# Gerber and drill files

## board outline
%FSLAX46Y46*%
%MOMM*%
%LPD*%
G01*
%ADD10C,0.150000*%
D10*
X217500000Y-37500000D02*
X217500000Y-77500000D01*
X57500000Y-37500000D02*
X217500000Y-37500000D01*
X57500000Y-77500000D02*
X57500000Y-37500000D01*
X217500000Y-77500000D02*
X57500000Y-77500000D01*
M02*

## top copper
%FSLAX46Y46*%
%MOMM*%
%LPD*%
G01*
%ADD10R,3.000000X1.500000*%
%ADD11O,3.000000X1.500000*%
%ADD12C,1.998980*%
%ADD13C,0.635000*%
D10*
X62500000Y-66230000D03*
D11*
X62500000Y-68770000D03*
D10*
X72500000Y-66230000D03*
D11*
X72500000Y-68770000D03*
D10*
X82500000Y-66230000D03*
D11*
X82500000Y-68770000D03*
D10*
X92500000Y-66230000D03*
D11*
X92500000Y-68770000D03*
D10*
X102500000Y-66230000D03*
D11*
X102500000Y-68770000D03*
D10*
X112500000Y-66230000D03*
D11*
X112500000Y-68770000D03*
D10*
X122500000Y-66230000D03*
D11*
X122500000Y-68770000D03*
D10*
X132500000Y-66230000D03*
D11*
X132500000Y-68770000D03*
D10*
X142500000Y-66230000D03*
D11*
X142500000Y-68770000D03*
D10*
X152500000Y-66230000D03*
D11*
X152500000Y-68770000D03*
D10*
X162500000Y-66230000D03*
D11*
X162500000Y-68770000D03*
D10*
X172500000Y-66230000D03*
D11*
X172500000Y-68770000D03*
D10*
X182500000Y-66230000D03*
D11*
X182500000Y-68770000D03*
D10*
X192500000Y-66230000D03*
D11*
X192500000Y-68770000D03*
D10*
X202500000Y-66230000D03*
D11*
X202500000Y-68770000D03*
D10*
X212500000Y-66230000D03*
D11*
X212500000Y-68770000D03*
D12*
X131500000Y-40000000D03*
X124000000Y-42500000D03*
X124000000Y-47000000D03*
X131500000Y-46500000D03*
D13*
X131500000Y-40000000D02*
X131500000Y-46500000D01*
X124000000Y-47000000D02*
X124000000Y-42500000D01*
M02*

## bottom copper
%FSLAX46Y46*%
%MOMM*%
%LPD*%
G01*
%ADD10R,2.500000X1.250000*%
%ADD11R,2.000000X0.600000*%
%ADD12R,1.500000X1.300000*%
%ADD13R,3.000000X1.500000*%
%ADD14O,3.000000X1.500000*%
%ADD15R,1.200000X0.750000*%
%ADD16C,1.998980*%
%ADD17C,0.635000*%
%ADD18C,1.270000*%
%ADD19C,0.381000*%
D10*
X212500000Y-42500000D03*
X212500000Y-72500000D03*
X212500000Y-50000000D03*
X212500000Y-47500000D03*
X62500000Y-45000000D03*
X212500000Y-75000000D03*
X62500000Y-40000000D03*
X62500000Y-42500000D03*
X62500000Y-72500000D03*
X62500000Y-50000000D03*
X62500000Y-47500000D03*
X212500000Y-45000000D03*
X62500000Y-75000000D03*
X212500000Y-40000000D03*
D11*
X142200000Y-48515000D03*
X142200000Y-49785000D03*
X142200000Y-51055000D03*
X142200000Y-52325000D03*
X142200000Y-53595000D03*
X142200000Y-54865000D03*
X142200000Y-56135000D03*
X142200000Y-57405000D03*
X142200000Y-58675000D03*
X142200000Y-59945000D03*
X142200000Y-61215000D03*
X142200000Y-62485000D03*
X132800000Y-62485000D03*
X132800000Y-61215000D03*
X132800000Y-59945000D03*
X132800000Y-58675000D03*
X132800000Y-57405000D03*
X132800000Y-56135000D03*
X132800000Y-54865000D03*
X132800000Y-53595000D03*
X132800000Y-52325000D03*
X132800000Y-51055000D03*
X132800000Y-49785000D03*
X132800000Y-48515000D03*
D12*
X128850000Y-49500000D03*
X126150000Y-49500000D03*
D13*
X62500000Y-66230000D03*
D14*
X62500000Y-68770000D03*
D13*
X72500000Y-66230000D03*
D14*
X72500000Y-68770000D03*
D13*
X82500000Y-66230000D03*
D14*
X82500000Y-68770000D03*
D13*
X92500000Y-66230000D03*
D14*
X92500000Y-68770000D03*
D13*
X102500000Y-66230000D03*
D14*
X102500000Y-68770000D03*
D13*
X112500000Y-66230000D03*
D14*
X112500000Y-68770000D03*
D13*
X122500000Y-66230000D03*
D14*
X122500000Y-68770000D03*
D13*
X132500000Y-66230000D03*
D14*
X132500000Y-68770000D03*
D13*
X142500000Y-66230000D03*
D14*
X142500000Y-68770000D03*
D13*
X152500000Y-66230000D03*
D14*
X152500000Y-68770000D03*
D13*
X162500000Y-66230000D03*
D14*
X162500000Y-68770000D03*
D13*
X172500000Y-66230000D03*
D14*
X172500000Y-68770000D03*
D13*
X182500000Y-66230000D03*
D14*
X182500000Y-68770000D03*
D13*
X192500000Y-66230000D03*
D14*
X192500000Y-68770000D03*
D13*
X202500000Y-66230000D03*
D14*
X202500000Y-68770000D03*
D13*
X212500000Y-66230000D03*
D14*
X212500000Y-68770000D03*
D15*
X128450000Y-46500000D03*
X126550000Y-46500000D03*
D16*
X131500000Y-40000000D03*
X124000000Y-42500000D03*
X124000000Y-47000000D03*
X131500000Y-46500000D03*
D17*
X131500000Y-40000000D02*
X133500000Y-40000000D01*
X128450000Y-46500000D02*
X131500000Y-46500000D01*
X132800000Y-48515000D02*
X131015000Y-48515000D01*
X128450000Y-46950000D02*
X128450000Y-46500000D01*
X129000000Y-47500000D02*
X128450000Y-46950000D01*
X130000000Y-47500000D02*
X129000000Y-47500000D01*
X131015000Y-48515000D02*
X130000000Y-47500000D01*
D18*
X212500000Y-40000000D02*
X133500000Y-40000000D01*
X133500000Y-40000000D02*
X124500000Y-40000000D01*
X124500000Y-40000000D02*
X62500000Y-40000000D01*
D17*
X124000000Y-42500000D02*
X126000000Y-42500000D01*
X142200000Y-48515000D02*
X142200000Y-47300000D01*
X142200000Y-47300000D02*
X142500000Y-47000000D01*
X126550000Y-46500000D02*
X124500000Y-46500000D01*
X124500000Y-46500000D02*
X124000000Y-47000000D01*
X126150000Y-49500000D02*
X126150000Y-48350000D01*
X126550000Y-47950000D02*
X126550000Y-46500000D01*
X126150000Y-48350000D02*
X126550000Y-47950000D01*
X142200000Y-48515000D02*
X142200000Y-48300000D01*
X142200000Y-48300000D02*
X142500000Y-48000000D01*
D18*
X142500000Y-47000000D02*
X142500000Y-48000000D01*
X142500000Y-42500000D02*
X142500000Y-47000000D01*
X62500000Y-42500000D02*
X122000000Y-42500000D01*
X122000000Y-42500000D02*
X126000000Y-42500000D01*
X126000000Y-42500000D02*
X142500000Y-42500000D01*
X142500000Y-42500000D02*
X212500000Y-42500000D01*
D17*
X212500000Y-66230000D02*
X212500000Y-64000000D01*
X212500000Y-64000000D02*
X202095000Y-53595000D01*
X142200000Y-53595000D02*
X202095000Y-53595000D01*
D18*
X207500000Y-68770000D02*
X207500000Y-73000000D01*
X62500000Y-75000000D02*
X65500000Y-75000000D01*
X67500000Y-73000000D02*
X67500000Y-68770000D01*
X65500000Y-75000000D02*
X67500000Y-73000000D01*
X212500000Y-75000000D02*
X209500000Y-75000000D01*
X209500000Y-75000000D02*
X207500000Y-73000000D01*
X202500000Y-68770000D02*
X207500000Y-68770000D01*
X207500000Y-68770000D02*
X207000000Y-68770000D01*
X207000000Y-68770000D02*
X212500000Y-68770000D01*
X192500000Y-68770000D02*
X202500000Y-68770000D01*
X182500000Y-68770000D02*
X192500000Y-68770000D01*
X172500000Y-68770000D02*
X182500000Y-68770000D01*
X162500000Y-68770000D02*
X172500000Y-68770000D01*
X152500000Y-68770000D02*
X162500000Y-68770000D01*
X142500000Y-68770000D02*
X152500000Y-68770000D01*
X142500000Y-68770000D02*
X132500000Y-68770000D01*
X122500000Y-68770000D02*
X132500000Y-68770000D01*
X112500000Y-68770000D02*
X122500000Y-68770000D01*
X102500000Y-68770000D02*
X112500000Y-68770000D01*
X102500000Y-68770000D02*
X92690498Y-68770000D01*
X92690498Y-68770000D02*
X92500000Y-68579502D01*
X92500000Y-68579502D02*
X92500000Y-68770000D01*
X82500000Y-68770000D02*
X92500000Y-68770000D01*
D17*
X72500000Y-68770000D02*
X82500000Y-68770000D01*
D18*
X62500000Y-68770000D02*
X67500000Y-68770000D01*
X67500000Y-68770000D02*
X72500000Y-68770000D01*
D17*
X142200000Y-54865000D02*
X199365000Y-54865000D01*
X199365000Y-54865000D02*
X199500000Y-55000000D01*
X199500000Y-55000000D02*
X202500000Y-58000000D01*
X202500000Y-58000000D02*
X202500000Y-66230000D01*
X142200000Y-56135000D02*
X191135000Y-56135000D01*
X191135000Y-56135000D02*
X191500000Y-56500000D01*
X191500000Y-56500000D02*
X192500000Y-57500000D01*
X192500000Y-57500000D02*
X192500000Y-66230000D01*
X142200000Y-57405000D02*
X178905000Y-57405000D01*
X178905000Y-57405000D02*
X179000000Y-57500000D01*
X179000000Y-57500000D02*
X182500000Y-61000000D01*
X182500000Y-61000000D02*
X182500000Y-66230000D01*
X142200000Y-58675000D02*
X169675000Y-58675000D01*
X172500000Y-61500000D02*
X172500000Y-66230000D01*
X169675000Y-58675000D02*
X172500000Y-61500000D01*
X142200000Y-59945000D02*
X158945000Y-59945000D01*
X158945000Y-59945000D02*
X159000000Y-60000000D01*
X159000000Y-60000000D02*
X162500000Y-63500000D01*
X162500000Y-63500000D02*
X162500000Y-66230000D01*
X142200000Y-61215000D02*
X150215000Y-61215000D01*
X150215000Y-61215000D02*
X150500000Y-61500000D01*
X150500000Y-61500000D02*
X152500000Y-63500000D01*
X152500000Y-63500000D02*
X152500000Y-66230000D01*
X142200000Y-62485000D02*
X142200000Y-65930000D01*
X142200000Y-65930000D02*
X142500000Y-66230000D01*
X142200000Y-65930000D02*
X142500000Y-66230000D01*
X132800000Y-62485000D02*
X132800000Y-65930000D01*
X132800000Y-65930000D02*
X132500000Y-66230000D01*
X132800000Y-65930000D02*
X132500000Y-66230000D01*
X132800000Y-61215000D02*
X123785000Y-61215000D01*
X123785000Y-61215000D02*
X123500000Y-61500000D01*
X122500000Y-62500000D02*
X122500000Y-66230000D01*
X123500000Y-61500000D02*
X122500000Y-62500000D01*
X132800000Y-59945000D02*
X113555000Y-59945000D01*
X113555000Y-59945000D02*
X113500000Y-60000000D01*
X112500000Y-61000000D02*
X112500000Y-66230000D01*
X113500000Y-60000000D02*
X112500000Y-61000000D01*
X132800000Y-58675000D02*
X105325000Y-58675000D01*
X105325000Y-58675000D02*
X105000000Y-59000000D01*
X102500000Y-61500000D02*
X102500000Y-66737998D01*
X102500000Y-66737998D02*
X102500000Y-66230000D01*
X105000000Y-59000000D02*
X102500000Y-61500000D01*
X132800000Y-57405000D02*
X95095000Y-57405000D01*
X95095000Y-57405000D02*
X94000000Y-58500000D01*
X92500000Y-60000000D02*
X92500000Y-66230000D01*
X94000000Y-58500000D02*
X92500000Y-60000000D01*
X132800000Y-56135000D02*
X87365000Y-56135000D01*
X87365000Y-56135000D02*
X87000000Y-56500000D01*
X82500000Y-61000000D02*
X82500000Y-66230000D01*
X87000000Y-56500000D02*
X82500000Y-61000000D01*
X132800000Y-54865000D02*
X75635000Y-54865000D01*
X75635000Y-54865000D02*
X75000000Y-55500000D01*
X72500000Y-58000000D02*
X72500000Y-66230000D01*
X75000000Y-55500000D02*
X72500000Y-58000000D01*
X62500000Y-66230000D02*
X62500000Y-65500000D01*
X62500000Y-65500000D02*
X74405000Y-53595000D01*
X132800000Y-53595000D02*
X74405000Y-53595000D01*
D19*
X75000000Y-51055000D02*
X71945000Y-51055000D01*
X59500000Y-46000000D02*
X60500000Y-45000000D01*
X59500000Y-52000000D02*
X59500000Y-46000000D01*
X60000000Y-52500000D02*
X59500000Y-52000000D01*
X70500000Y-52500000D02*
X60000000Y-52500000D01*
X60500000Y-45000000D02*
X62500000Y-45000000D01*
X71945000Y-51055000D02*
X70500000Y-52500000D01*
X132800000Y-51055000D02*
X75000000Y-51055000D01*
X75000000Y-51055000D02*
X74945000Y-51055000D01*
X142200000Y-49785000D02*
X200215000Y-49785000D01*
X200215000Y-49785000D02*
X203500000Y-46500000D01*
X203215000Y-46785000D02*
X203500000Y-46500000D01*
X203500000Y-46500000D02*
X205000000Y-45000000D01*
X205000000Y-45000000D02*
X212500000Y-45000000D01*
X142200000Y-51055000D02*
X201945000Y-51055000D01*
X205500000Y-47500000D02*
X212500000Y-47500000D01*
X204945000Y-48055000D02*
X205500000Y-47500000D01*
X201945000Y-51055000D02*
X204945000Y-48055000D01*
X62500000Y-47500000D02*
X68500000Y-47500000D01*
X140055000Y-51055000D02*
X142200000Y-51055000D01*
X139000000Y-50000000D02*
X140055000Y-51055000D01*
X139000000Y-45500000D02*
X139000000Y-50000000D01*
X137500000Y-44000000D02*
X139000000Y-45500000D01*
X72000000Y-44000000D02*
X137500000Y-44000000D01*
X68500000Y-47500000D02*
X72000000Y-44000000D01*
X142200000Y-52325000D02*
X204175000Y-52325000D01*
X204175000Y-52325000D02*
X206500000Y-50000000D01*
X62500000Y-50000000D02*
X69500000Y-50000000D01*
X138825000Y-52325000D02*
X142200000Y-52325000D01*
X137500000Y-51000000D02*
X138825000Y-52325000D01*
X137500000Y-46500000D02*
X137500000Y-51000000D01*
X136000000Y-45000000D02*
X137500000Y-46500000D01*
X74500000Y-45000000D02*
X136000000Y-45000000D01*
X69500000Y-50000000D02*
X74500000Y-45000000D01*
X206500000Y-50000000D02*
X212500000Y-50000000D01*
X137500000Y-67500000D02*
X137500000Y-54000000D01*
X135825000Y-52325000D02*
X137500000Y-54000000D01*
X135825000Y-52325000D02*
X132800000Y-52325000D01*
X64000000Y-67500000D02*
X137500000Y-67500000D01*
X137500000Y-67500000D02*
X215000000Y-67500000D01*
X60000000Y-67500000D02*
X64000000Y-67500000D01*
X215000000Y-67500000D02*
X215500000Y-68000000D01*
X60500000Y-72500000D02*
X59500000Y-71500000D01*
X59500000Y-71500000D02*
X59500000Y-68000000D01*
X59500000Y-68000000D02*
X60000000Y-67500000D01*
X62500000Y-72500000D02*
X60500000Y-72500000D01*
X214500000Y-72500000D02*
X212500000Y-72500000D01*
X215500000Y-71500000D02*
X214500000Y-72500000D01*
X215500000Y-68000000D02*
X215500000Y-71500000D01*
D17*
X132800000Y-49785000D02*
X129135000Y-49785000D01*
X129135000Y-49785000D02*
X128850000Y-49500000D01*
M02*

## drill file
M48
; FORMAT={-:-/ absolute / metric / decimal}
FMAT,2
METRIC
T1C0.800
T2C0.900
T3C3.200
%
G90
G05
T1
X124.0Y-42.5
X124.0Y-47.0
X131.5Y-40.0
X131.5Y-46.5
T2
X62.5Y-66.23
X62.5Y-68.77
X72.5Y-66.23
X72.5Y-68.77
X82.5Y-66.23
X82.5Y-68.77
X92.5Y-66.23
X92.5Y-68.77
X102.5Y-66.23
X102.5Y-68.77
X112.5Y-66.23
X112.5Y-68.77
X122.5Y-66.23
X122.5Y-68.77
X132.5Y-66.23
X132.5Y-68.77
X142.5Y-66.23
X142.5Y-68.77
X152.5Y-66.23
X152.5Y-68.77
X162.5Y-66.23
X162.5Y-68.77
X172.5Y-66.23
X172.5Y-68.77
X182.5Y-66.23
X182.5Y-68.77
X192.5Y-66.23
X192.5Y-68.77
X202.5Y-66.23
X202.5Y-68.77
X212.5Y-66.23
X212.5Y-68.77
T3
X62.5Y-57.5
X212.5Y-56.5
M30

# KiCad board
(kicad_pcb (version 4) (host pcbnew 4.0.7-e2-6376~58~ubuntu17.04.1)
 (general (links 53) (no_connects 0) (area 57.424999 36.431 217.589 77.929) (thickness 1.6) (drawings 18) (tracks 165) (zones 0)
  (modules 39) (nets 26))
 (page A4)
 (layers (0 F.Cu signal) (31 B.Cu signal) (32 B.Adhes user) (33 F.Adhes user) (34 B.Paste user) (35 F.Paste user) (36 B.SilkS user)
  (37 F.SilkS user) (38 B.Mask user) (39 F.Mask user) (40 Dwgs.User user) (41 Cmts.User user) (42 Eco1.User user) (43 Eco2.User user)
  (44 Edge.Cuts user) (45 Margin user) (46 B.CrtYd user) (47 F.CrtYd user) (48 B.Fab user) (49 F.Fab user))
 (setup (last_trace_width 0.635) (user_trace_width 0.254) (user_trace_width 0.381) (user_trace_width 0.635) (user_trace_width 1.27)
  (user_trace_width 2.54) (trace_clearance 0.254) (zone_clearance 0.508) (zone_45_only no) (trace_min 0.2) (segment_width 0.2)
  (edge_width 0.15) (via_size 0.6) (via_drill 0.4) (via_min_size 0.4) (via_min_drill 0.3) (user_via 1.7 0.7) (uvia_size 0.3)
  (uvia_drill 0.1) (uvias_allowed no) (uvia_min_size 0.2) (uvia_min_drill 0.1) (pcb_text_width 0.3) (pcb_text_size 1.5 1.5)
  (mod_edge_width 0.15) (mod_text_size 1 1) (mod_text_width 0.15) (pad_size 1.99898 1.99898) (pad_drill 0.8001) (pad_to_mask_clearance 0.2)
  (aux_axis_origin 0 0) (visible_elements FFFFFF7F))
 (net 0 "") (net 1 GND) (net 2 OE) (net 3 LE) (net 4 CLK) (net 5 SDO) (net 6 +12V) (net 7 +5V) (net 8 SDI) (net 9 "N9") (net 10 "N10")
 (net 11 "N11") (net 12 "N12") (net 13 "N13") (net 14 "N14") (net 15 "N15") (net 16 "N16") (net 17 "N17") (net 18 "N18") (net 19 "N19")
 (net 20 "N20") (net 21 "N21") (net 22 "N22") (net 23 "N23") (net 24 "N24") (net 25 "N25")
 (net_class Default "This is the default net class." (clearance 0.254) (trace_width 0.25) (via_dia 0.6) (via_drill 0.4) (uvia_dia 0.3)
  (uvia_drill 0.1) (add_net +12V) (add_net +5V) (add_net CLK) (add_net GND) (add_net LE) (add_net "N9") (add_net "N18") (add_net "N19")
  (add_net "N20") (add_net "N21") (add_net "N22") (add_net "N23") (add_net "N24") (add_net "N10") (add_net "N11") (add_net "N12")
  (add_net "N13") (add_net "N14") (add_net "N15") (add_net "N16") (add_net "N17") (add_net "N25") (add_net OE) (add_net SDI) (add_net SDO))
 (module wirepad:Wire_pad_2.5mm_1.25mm (layer B.Cu) (at 212.5 42.5 180)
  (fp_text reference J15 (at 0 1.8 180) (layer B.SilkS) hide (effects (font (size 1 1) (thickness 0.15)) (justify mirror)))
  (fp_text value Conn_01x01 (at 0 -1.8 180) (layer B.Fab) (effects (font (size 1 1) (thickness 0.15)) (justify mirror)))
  (pad 1 smd rect (at 0 0 180) (size 2.5 1.25) (layers B.Cu B.Mask) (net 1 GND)))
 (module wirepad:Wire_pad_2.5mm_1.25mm (layer B.Cu) (at 212.5 72.5 180)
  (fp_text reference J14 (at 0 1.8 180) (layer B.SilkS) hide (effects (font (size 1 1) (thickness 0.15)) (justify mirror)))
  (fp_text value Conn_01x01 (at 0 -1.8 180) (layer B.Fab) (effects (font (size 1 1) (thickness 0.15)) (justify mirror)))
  (pad 1 smd rect (at 0 0 180) (size 2.5 1.25) (layers B.Cu B.Mask) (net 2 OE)))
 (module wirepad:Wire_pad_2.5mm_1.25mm (layer B.Cu) (at 212.5 50 180)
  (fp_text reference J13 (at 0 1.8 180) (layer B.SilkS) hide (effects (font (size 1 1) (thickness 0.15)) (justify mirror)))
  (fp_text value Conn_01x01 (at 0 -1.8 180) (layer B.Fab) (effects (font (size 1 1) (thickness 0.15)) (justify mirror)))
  (pad 1 smd rect (at 0 0 180) (size 2.5 1.25) (layers B.Cu B.Mask) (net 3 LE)))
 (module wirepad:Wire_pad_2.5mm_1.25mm (layer B.Cu) (at 212.5 47.5 180)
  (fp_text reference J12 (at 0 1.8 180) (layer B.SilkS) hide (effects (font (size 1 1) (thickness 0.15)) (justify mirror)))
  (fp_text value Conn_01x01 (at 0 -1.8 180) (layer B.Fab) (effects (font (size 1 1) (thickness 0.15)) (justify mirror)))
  (pad 1 smd rect (at 0 0 180) (size 2.5 1.25) (layers B.Cu B.Mask) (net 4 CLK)))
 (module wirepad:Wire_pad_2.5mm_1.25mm (layer B.Cu) (at 62.5 45 180)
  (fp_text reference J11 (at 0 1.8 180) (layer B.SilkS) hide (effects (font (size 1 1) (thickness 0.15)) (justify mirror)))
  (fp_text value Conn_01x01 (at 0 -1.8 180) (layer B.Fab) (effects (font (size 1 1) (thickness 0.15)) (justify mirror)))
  (pad 1 smd rect (at 0 0 180) (size 2.5 1.25) (layers B.Cu B.Mask) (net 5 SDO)))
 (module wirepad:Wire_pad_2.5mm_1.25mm (layer B.Cu) (at 212.5 75 180)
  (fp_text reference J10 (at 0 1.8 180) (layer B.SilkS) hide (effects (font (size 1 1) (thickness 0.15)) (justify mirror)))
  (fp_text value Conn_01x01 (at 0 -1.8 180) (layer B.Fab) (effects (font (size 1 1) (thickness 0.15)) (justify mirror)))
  (pad 1 smd rect (at 0 0 180) (size 2.5 1.25) (layers B.Cu B.Mask) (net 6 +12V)))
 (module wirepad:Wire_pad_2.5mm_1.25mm (layer B.Cu) (at 62.5 40 180)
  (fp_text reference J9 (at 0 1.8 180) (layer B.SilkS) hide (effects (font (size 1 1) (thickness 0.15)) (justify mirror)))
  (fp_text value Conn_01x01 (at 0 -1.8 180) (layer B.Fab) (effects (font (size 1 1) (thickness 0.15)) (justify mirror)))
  (pad 1 smd rect (at 0 0 180) (size 2.5 1.25) (layers B.Cu B.Mask) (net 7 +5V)))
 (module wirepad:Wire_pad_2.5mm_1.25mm (layer B.Cu) (at 62.5 42.5 180)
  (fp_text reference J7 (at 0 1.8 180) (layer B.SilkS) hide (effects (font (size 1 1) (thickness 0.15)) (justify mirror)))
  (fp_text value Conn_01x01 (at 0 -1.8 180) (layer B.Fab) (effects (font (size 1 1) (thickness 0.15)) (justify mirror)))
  (pad 1 smd rect (at 0 0 180) (size 2.5 1.25) (layers B.Cu B.Mask) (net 1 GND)))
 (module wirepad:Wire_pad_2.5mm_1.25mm (layer B.Cu) (at 62.5 72.5 180)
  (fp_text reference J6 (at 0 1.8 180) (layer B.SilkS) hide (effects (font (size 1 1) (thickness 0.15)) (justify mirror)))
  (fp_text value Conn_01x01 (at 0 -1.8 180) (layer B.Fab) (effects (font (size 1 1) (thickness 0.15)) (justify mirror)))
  (pad 1 smd rect (at 0 0 180) (size 2.5 1.25) (layers B.Cu B.Mask) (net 2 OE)))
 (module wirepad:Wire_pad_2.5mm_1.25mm (layer B.Cu) (at 62.5 50 180)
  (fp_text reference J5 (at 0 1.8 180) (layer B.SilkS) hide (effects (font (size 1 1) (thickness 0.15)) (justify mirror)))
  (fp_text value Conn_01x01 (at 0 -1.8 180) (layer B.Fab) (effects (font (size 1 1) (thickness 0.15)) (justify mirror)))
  (pad 1 smd rect (at 0 0 180) (size 2.5 1.25) (layers B.Cu B.Mask) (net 3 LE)))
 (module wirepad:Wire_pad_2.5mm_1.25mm (layer B.Cu) (at 62.5 47.5 180)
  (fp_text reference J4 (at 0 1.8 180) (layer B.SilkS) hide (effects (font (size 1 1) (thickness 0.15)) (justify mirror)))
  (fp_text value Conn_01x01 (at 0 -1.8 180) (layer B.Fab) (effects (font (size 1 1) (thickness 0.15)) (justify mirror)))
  (pad 1 smd rect (at 0 0 180) (size 2.5 1.25) (layers B.Cu B.Mask) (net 4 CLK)))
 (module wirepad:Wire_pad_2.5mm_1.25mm (layer B.Cu) (at 212.5 45 180)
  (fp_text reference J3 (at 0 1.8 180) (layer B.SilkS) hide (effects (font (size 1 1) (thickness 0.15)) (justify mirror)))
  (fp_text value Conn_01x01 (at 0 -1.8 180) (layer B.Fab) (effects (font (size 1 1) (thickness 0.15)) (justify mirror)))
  (pad 1 smd rect (at 0 0 180) (size 2.5 1.25) (layers B.Cu B.Mask) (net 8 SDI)))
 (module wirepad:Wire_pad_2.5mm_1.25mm (layer B.Cu) (at 62.5 75 180)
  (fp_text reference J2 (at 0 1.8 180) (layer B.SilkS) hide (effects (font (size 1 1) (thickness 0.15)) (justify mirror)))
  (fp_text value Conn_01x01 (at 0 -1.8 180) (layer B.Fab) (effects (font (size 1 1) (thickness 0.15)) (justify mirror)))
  (pad 1 smd rect (at 0 0 180) (size 2.5 1.25) (layers B.Cu B.Mask) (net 6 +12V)))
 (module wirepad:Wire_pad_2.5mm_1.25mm (layer B.Cu) (at 212.5 40 180)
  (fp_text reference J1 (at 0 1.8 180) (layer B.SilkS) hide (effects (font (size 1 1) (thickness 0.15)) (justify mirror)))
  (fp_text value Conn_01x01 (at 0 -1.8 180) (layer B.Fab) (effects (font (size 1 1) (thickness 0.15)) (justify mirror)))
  (pad 1 smd rect (at 0 0 180) (size 2.5 1.25) (layers B.Cu B.Mask) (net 7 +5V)))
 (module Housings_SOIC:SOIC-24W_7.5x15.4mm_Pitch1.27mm (layer B.Cu) (at 137.5 55.5 180)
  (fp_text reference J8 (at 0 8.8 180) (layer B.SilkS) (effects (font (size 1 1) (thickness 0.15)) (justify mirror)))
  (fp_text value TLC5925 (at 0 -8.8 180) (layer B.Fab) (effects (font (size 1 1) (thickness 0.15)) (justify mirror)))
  (pad 1 smd rect (at -4.7 6.985 180) (size 2 0.6) (layers B.Cu B.Paste B.Mask) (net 1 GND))
  (pad 2 smd rect (at -4.7 5.715 180) (size 2 0.6) (layers B.Cu B.Paste B.Mask) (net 8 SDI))
  (pad 3 smd rect (at -4.7 4.445 180) (size 2 0.6) (layers B.Cu B.Paste B.Mask) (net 4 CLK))
  (pad 4 smd rect (at -4.7 3.175 180) (size 2 0.6) (layers B.Cu B.Paste B.Mask) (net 3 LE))
  (pad 5 smd rect (at -4.7 1.905 180) (size 2 0.6) (layers B.Cu B.Paste B.Mask) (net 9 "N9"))
  (pad 6 smd rect (at -4.7 0.635 180) (size 2 0.6) (layers B.Cu B.Paste B.Mask) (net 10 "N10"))
  (pad 7 smd rect (at -4.7 -0.635 180) (size 2 0.6) (layers B.Cu B.Paste B.Mask) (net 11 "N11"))
  (pad 8 smd rect (at -4.7 -1.905 180) (size 2 0.6) (layers B.Cu B.Paste B.Mask) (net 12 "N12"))
  (pad 9 smd rect (at -4.7 -3.175 180) (size 2 0.6) (layers B.Cu B.Paste B.Mask) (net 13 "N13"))
  (pad 10 smd rect (at -4.7 -4.445 180) (size 2 0.6) (layers B.Cu B.Paste B.Mask) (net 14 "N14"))
  (pad 11 smd rect (at -4.7 -5.715 180) (size 2 0.6) (layers B.Cu B.Paste B.Mask) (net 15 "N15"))
  (pad 12 smd rect (at -4.7 -6.985 180) (size 2 0.6) (layers B.Cu B.Paste B.Mask) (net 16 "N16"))
  (pad 13 smd rect (at 4.7 -6.985 180) (size 2 0.6) (layers B.Cu B.Paste B.Mask) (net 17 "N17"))
  (pad 14 smd rect (at 4.7 -5.715 180) (size 2 0.6) (layers B.Cu B.Paste B.Mask) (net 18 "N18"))
  (pad 15 smd rect (at 4.7 -4.445 180) (size 2 0.6) (layers B.Cu B.Paste B.Mask) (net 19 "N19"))
  (pad 16 smd rect (at 4.7 -3.175 180) (size 2 0.6) (layers B.Cu B.Paste B.Mask) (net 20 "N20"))
  (pad 17 smd rect (at 4.7 -1.905 180) (size 2 0.6) (layers B.Cu B.Paste B.Mask) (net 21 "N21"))
  (pad 18 smd rect (at 4.7 -0.635 180) (size 2 0.6) (layers B.Cu B.Paste B.Mask) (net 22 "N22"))
  (pad 19 smd rect (at 4.7 0.635 180) (size 2 0.6) (layers B.Cu B.Paste B.Mask) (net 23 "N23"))
  (pad 20 smd rect (at 4.7 1.905 180) (size 2 0.6) (layers B.Cu B.Paste B.Mask) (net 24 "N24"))
  (pad 21 smd rect (at 4.7 3.175 180) (size 2 0.6) (layers B.Cu B.Paste B.Mask) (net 2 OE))
  (pad 22 smd rect (at 4.7 4.445 180) (size 2 0.6) (layers B.Cu B.Paste B.Mask) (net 5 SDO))
  (pad 23 smd rect (at 4.7 5.715 180) (size 2 0.6) (layers B.Cu B.Paste B.Mask) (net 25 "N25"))
  (pad 24 smd rect (at 4.7 6.985 180) (size 2 0.6) (layers B.Cu B.Paste B.Mask) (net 7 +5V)))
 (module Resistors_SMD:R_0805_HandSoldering (layer B.Cu) (at 127.5 49.5 180)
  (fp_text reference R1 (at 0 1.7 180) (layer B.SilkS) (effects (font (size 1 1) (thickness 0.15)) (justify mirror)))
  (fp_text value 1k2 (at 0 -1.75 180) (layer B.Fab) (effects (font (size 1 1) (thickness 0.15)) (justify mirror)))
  (pad 1 smd rect (at -1.35 0 180) (size 1.5 1.3) (layers B.Cu B.Paste B.Mask) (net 25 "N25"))
  (pad 2 smd rect (at 1.35 0 180) (size 1.5 1.3) (layers B.Cu B.Paste B.Mask) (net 1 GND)))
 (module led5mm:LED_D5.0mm (layer F.Cu) (at 62.5 67.5 270)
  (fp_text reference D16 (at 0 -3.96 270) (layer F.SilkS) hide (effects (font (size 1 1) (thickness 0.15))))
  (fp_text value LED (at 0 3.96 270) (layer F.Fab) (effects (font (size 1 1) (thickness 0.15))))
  (pad 1 thru_hole rect (at -1.27 0 270) (size 1.5 3) (drill 0.9) (layers *.Cu *.Mask) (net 24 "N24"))
  (pad 2 thru_hole oval (at 1.27 0 270) (size 1.5 3) (drill 0.9) (layers *.Cu *.Mask) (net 6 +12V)))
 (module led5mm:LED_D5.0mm (layer F.Cu) (at 72.5 67.5 270)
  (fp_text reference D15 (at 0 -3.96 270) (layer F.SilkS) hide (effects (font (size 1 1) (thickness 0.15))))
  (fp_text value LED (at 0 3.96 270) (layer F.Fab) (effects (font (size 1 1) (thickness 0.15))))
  (pad 1 thru_hole rect (at -1.27 0 270) (size 1.5 3) (drill 0.9) (layers *.Cu *.Mask) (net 23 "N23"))
  (pad 2 thru_hole oval (at 1.27 0 270) (size 1.5 3) (drill 0.9) (layers *.Cu *.Mask) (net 6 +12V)))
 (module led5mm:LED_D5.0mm (layer F.Cu) (at 82.5 67.5 270)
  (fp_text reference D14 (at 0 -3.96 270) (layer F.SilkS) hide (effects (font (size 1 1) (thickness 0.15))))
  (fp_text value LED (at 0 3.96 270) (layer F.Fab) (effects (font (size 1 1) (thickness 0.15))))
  (pad 1 thru_hole rect (at -1.27 0 270) (size 1.5 3) (drill 0.9) (layers *.Cu *.Mask) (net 22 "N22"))
  (pad 2 thru_hole oval (at 1.27 0 270) (size 1.5 3) (drill 0.9) (layers *.Cu *.Mask) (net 6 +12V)))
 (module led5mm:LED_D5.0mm (layer F.Cu) (at 92.5 67.5 270)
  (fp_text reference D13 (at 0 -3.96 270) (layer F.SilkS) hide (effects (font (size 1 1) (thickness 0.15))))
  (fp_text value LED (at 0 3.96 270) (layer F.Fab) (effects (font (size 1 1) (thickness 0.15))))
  (pad 1 thru_hole rect (at -1.27 0 270) (size 1.5 3) (drill 0.9) (layers *.Cu *.Mask) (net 21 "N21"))
  (pad 2 thru_hole oval (at 1.27 0 270) (size 1.5 3) (drill 0.9) (layers *.Cu *.Mask) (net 6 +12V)))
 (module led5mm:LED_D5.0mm (layer F.Cu) (at 102.5 67.5 270)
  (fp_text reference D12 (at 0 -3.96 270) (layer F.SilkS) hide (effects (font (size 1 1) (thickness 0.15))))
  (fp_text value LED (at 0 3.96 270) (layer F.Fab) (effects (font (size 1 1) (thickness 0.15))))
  (pad 1 thru_hole rect (at -1.27 0 270) (size 1.5 3) (drill 0.9) (layers *.Cu *.Mask) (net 20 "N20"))
  (pad 2 thru_hole oval (at 1.27 0 270) (size 1.5 3) (drill 0.9) (layers *.Cu *.Mask) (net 6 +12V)))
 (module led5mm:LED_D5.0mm (layer F.Cu) (at 112.5 67.5 270)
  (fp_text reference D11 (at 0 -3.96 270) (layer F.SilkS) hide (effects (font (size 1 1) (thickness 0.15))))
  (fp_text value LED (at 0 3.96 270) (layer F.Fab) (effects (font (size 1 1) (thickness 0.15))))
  (pad 1 thru_hole rect (at -1.27 0 270) (size 1.5 3) (drill 0.9) (layers *.Cu *.Mask) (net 19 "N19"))
  (pad 2 thru_hole oval (at 1.27 0 270) (size 1.5 3) (drill 0.9) (layers *.Cu *.Mask) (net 6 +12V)))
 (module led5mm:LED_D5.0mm (layer F.Cu) (at 122.5 67.5 270)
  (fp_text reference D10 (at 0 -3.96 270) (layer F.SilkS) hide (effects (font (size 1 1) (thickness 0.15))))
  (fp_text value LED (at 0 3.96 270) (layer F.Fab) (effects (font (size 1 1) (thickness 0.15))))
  (pad 1 thru_hole rect (at -1.27 0 270) (size 1.5 3) (drill 0.9) (layers *.Cu *.Mask) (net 18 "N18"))
  (pad 2 thru_hole oval (at 1.27 0 270) (size 1.5 3) (drill 0.9) (layers *.Cu *.Mask) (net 6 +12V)))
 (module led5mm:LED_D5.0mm (layer F.Cu) (at 132.5 67.5 270)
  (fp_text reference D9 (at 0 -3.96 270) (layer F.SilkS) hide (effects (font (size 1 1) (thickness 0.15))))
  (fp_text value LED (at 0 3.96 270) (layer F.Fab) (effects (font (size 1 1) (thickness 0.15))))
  (pad 1 thru_hole rect (at -1.27 0 270) (size 1.5 3) (drill 0.9) (layers *.Cu *.Mask) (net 17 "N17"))
  (pad 2 thru_hole oval (at 1.27 0 270) (size 1.5 3) (drill 0.9) (layers *.Cu *.Mask) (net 6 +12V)))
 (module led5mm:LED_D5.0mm (layer F.Cu) (at 142.5 67.5 270)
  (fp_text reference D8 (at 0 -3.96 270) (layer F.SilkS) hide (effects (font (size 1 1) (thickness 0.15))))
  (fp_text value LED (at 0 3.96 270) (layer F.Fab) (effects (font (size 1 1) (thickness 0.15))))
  (pad 1 thru_hole rect (at -1.27 0 270) (size 1.5 3) (drill 0.9) (layers *.Cu *.Mask) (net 16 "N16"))
  (pad 2 thru_hole oval (at 1.27 0 270) (size 1.5 3) (drill 0.9) (layers *.Cu *.Mask) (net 6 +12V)))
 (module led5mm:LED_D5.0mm (layer F.Cu) (at 152.5 67.5 270)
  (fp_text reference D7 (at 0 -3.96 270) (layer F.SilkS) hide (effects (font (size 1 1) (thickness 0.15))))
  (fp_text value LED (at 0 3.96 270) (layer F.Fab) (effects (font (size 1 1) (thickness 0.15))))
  (pad 1 thru_hole rect (at -1.27 0 270) (size 1.5 3) (drill 0.9) (layers *.Cu *.Mask) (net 15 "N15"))
  (pad 2 thru_hole oval (at 1.27 0 270) (size 1.5 3) (drill 0.9) (layers *.Cu *.Mask) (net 6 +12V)))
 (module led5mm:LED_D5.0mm (layer F.Cu) (at 162.5 67.5 270)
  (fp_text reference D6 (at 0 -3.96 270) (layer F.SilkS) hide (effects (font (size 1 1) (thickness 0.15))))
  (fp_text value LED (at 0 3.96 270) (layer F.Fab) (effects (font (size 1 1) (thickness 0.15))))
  (pad 1 thru_hole rect (at -1.27 0 270) (size 1.5 3) (drill 0.9) (layers *.Cu *.Mask) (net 14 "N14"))
  (pad 2 thru_hole oval (at 1.27 0 270) (size 1.5 3) (drill 0.9) (layers *.Cu *.Mask) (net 6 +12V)))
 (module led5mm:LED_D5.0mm (layer F.Cu) (at 172.5 67.5 270)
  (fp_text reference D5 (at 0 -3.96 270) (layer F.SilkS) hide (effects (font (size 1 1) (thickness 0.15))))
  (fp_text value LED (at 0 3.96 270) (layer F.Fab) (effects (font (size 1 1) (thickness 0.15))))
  (pad 1 thru_hole rect (at -1.27 0 270) (size 1.5 3) (drill 0.9) (layers *.Cu *.Mask) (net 13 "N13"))
  (pad 2 thru_hole oval (at 1.27 0 270) (size 1.5 3) (drill 0.9) (layers *.Cu *.Mask) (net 6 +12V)))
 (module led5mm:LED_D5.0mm (layer F.Cu) (at 182.5 67.5 270)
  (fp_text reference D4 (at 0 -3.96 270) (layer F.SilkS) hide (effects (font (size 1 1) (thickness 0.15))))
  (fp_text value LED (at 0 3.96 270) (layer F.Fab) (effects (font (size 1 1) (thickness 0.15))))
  (pad 1 thru_hole rect (at -1.27 0 270) (size 1.5 3) (drill 0.9) (layers *.Cu *.Mask) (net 12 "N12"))
  (pad 2 thru_hole oval (at 1.27 0 270) (size 1.5 3) (drill 0.9) (layers *.Cu *.Mask) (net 6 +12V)))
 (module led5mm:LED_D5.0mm (layer F.Cu) (at 192.5 67.5 270)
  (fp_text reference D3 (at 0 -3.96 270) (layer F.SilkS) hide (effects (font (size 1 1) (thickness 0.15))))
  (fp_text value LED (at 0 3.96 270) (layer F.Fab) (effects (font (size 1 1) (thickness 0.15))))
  (pad 1 thru_hole rect (at -1.27 0 270) (size 1.5 3) (drill 0.9) (layers *.Cu *.Mask) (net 11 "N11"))
  (pad 2 thru_hole oval (at 1.27 0 270) (size 1.5 3) (drill 0.9) (layers *.Cu *.Mask) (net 6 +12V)))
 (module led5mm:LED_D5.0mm (layer F.Cu) (at 202.5 67.5 270)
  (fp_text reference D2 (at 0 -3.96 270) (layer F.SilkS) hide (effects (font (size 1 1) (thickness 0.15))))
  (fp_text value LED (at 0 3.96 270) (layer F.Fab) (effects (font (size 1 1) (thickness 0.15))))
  (pad 1 thru_hole rect (at -1.27 0 270) (size 1.5 3) (drill 0.9) (layers *.Cu *.Mask) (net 10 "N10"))
  (pad 2 thru_hole oval (at 1.27 0 270) (size 1.5 3) (drill 0.9) (layers *.Cu *.Mask) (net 6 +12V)))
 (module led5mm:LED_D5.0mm (layer F.Cu) (at 212.5 67.5 270)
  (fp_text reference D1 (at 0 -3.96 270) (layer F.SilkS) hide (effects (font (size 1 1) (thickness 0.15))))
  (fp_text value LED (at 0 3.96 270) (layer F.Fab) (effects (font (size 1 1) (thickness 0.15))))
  (pad 1 thru_hole rect (at -1.27 0 270) (size 1.5 3) (drill 0.9) (layers *.Cu *.Mask) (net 9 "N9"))
  (pad 2 thru_hole oval (at 1.27 0 270) (size 1.5 3) (drill 0.9) (layers *.Cu *.Mask) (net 6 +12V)))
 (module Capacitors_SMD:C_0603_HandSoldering (layer B.Cu) (at 127.5 46.5 180)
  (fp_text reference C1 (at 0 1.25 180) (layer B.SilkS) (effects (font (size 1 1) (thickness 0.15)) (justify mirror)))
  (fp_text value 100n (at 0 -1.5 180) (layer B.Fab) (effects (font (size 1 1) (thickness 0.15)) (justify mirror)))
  (pad 1 smd rect (at -0.95 0 180) (size 1.2 0.75) (layers B.Cu B.Paste B.Mask) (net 7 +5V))
  (pad 2 smd rect (at 0.95 0 180) (size 1.2 0.75) (layers B.Cu B.Paste B.Mask) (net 1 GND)))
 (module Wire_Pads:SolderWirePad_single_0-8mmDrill (layer F.Cu) (at 131.5 40)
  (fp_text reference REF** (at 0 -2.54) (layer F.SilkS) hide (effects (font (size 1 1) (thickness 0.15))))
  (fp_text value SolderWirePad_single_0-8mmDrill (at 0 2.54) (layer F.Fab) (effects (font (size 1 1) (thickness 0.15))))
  (pad 1 thru_hole circle (at 0 0) (size 1.99898 1.99898) (drill 0.8001) (layers *.Cu *.Mask) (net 7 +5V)))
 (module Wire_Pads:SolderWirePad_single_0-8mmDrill (layer F.Cu) (at 124 42.5)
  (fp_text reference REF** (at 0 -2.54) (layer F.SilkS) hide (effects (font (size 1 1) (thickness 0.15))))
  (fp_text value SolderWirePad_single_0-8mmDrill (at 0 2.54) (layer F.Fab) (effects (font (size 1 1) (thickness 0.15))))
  (pad 1 thru_hole circle (at 0 0) (size 1.99898 1.99898) (drill 0.8001) (layers *.Cu *.Mask) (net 1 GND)))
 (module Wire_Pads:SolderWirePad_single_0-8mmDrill (layer F.Cu) (at 124 47)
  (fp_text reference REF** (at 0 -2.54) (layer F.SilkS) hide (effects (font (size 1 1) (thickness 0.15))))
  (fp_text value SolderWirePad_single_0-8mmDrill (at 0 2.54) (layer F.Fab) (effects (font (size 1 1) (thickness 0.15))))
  (pad 1 thru_hole circle (at 0 0) (size 1.99898 1.99898) (drill 0.8001) (layers *.Cu *.Mask) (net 1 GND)))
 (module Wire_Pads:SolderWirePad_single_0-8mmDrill (layer F.Cu) (at 131.5 46.5)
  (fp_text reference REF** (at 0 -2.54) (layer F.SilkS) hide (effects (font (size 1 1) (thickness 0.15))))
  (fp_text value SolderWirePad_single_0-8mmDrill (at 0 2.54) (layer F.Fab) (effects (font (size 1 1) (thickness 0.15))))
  (pad 1 thru_hole circle (at 0 0) (size 1.99898 1.99898) (drill 0.8001) (layers *.Cu *.Mask) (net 7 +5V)))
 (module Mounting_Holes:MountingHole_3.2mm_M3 (layer F.Cu) (at 212.5 56.5)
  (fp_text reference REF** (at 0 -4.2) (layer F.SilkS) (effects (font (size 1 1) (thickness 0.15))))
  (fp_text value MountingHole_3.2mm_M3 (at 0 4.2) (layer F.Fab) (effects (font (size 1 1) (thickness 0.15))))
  (pad 1 np_thru_hole circle (at 0 0) (size 3.2 3.2) (drill 3.2) (layers *.Cu *.Mask)))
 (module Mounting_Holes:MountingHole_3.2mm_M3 (layer F.Cu) (at 62.5 57.5)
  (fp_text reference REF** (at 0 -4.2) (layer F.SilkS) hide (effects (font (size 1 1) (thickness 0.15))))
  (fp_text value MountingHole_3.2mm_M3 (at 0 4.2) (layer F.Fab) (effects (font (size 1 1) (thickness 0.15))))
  (pad 1 np_thru_hole circle (at 0 0) (size 3.2 3.2) (drill 3.2) (layers *.Cu *.Mask)))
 (gr_line (start 217.5 37.5) (end 217.5 77.5) (angle 90) (layer Edge.Cuts) (width 0.15))
 (gr_line (start 57.5 37.5) (end 217.5 37.5) (angle 90) (layer Edge.Cuts) (width 0.15))
 (gr_line (start 57.5 77.5) (end 57.5 37.5) (angle 90) (layer Edge.Cuts) (width 0.15))
 (gr_line (start 217.5 77.5) (end 57.5 77.5) (angle 90) (layer Edge.Cuts) (width 0.15))
 (segment (start 131.5 40) (end 133.5 40) (width 0.635) (layer B.Cu) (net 7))
 (segment (start 131.5 40) (end 131.5 46.5) (width 0.635) (layer F.Cu) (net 7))
 (segment (start 128.45 46.5) (end 131.5 46.5) (width 0.635) (layer B.Cu) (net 7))
 (segment (start 132.8 48.515) (end 131.015 48.515) (width 0.635) (layer B.Cu) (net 7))
 (segment (start 128.45 46.95) (end 128.45 46.5) (width 0.635) (layer B.Cu) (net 7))
 (segment (start 129 47.5) (end 128.45 46.95) (width 0.635) (layer B.Cu) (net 7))
 (segment (start 130 47.5) (end 129 47.5) (width 0.635) (layer B.Cu) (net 7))
 (segment (start 131.015 48.515) (end 130 47.5) (width 0.635) (layer B.Cu) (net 7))
 (segment (start 212.5 40) (end 133.5 40) (width 1.27) (layer B.Cu) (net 7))
 (segment (start 133.5 40) (end 124.5 40) (width 1.27) (layer B.Cu) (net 7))
 (segment (start 124.5 40) (end 62.5 40) (width 1.27) (layer B.Cu) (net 7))
 (segment (start 124 42.5) (end 126 42.5) (width 0.635) (layer B.Cu) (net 1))
 (segment (start 142.2 48.515) (end 142.2 47.3) (width 0.635) (layer B.Cu) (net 1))
 (segment (start 142.2 47.3) (end 142.5 47) (width 0.635) (layer B.Cu) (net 1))
 (segment (start 124 47) (end 124 42.5) (width 0.635) (layer F.Cu) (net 1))
 (segment (start 126.55 46.5) (end 124.5 46.5) (width 0.635) (layer B.Cu) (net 1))
 (segment (start 124.5 46.5) (end 124 47) (width 0.635) (layer B.Cu) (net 1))
 (segment (start 126.15 49.5) (end 126.15 48.35) (width 0.635) (layer B.Cu) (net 1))
 (segment (start 126.55 47.95) (end 126.55 46.5) (width 0.635) (layer B.Cu) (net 1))
 (segment (start 126.15 48.35) (end 126.55 47.95) (width 0.635) (layer B.Cu) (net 1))
 (segment (start 142.2 48.515) (end 142.2 48.3) (width 0.635) (layer B.Cu) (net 1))
 (segment (start 142.2 48.3) (end 142.5 48) (width 0.635) (layer B.Cu) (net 1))
 (segment (start 142.5 47) (end 142.5 48) (width 1.27) (layer B.Cu) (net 1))
 (segment (start 142.5 42.5) (end 142.5 47) (width 1.27) (layer B.Cu) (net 1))
 (segment (start 62.5 42.5) (end 122 42.5) (width 1.27) (layer B.Cu) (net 1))
 (segment (start 122 42.5) (end 126 42.5) (width 1.27) (layer B.Cu) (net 1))
 (segment (start 126 42.5) (end 142.5 42.5) (width 1.27) (layer B.Cu) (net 1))
 (segment (start 142.5 42.5) (end 212.5 42.5) (width 1.27) (layer B.Cu) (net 1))
 (segment (start 212.5 66.23) (end 212.5 64) (width 0.635) (layer B.Cu) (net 9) (status 400000))
 (segment (start 212.5 64) (end 202.095 53.595) (width 0.635) (layer B.Cu) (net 9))
 (segment (start 142.2 53.595) (end 202.095 53.595) (width 0.635) (layer B.Cu) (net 9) (status 400000))
 (segment (start 207.5 68.77) (end 207.5 73) (width 1.27) (layer B.Cu) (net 6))
 (segment (start 62.5 75) (end 65.5 75) (width 1.27) (layer B.Cu) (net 6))
 (segment (start 67.5 73) (end 67.5 68.77) (width 1.27) (layer B.Cu) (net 6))
 (segment (start 65.5 75) (end 67.5 73) (width 1.27) (layer B.Cu) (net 6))
 (segment (start 212.5 75) (end 209.5 75) (width 1.27) (layer B.Cu) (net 6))
 (segment (start 209.5 75) (end 207.5 73) (width 1.27) (layer B.Cu) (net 6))
 (segment (start 202.5 68.77) (end 207.5 68.77) (width 1.27) (layer B.Cu) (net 6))
 (segment (start 207.5 68.77) (end 207 68.77) (width 1.27) (layer B.Cu) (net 6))
 (segment (start 207 68.77) (end 212.5 68.77) (width 1.27) (layer B.Cu) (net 6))
 (segment (start 192.5 68.77) (end 202.5 68.77) (width 1.27) (layer B.Cu) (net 6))
 (segment (start 182.5 68.77) (end 192.5 68.77) (width 1.27) (layer B.Cu) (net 6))
 (segment (start 172.5 68.77) (end 182.5 68.77) (width 1.27) (layer B.Cu) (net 6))
 (segment (start 162.5 68.77) (end 172.5 68.77) (width 1.27) (layer B.Cu) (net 6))
 (segment (start 152.5 68.77) (end 162.5 68.77) (width 1.27) (layer B.Cu) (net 6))
 (segment (start 142.5 68.77) (end 152.5 68.77) (width 1.27) (layer B.Cu) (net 6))
 (segment (start 142.5 68.77) (end 132.5 68.77) (width 1.27) (layer B.Cu) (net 6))
 (segment (start 122.5 68.77) (end 132.5 68.77) (width 1.27) (layer B.Cu) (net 6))
 (segment (start 112.5 68.77) (end 122.5 68.77) (width 1.27) (layer B.Cu) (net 6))
 (segment (start 102.5 68.77) (end 112.5 68.77) (width 1.27) (layer B.Cu) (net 6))
 (segment (start 102.5 68.77) (end 92.690498 68.77) (width 1.27) (layer B.Cu) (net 6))
 (segment (start 92.690498 68.77) (end 92.5 68.579502) (width 1.27) (layer B.Cu) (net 6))
 (segment (start 92.5 68.579502) (end 92.5 68.77) (width 1.27) (layer B.Cu) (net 6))
 (segment (start 82.5 68.77) (end 92.5 68.77) (width 1.27) (layer B.Cu) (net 6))
 (segment (start 72.5 68.77) (end 82.5 68.77) (width 0.635) (layer B.Cu) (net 6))
 (segment (start 62.5 68.77) (end 67.5 68.77) (width 1.27) (layer B.Cu) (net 6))
 (segment (start 67.5 68.77) (end 72.5 68.77) (width 1.27) (layer B.Cu) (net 6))
 (segment (start 142.2 54.865) (end 199.365 54.865) (width 0.635) (layer B.Cu) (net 10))
 (segment (start 199.365 54.865) (end 199.5 55) (width 0.635) (layer B.Cu) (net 10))
 (segment (start 199.5 55) (end 202.5 58) (width 0.635) (layer B.Cu) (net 10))
 (segment (start 202.5 58) (end 202.5 66.23) (width 0.635) (layer B.Cu) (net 10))
 (segment (start 142.2 56.135) (end 191.135 56.135) (width 0.635) (layer B.Cu) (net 11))
 (segment (start 191.135 56.135) (end 191.5 56.5) (width 0.635) (layer B.Cu) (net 11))
 (segment (start 191.5 56.5) (end 192.5 57.5) (width 0.635) (layer B.Cu) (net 11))
 (segment (start 192.5 57.5) (end 192.5 66.23) (width 0.635) (layer B.Cu) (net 11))
 (segment (start 142.2 57.405) (end 178.905 57.405) (width 0.635) (layer B.Cu) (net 12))
 (segment (start 178.905 57.405) (end 179 57.5) (width 0.635) (layer B.Cu) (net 12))
 (segment (start 179 57.5) (end 182.5 61) (width 0.635) (layer B.Cu) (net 12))
 (segment (start 182.5 61) (end 182.5 66.23) (width 0.635) (layer B.Cu) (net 12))
 (segment (start 142.2 58.675) (end 169.675 58.675) (width 0.635) (layer B.Cu) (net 13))
 (segment (start 172.5 61.5) (end 172.5 66.23) (width 0.635) (layer B.Cu) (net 13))
 (segment (start 169.675 58.675) (end 172.5 61.5) (width 0.635) (layer B.Cu) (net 13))
 (segment (start 142.2 59.945) (end 158.945 59.945) (width 0.635) (layer B.Cu) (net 14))
 (segment (start 158.945 59.945) (end 159 60) (width 0.635) (layer B.Cu) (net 14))
 (segment (start 159 60) (end 162.5 63.5) (width 0.635) (layer B.Cu) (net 14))
 (segment (start 162.5 63.5) (end 162.5 66.23) (width 0.635) (layer B.Cu) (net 14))
 (segment (start 142.2 61.215) (end 150.215 61.215) (width 0.635) (layer B.Cu) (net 15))
 (segment (start 150.215 61.215) (end 150.5 61.5) (width 0.635) (layer B.Cu) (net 15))
 (segment (start 150.5 61.5) (end 152.5 63.5) (width 0.635) (layer B.Cu) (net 15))
 (segment (start 152.5 63.5) (end 152.5 66.23) (width 0.635) (layer B.Cu) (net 15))
 (segment (start 142.2 62.485) (end 142.2 65.93) (width 0.635) (layer B.Cu) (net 16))
 (segment (start 142.2 65.93) (end 142.5 66.23) (width 0.635) (layer B.Cu) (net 16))
 (segment (start 142.2 65.93) (end 142.5 66.23) (width 0.635) (layer B.Cu) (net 16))
 (segment (start 132.8 62.485) (end 132.8 65.93) (width 0.635) (layer B.Cu) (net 17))
 (segment (start 132.8 65.93) (end 132.5 66.23) (width 0.635) (layer B.Cu) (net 17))
 (segment (start 132.8 65.93) (end 132.5 66.23) (width 0.635) (layer B.Cu) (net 17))
 (segment (start 132.8 61.215) (end 123.785 61.215) (width 0.635) (layer B.Cu) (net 18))
 (segment (start 123.785 61.215) (end 123.5 61.5) (width 0.635) (layer B.Cu) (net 18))
 (segment (start 122.5 62.5) (end 122.5 66.23) (width 0.635) (layer B.Cu) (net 18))
 (segment (start 123.5 61.5) (end 122.5 62.5) (width 0.635) (layer B.Cu) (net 18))
 (segment (start 132.8 59.945) (end 113.555 59.945) (width 0.635) (layer B.Cu) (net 19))
 (segment (start 113.555 59.945) (end 113.5 60) (width 0.635) (layer B.Cu) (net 19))
 (segment (start 112.5 61) (end 112.5 66.23) (width 0.635) (layer B.Cu) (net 19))
 (segment (start 113.5 60) (end 112.5 61) (width 0.635) (layer B.Cu) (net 19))
 (segment (start 132.8 58.675) (end 105.325 58.675) (width 0.635) (layer B.Cu) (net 20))
 (segment (start 105.325 58.675) (end 105 59) (width 0.635) (layer B.Cu) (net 20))
 (segment (start 102.5 61.5) (end 102.5 66.737998) (width 0.635) (layer B.Cu) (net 20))
 (segment (start 102.5 66.737998) (end 102.5 66.23) (width 0.635) (layer B.Cu) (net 20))
 (segment (start 105 59) (end 102.5 61.5) (width 0.635) (layer B.Cu) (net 20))
 (segment (start 132.8 57.405) (end 95.095 57.405) (width 0.635) (layer B.Cu) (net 21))
 (segment (start 95.095 57.405) (end 94 58.5) (width 0.635) (layer B.Cu) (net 21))
 (segment (start 92.5 60) (end 92.5 66.23) (width 0.635) (layer B.Cu) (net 21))
 (segment (start 94 58.5) (end 92.5 60) (width 0.635) (layer B.Cu) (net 21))
 (segment (start 132.8 56.135) (end 87.365 56.135) (width 0.635) (layer B.Cu) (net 22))
 (segment (start 87.365 56.135) (end 87 56.5) (width 0.635) (layer B.Cu) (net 22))
 (segment (start 82.5 61) (end 82.5 66.23) (width 0.635) (layer B.Cu) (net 22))
 (segment (start 87 56.5) (end 82.5 61) (width 0.635) (layer B.Cu) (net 22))
 (segment (start 132.8 54.865) (end 75.635 54.865) (width 0.635) (layer B.Cu) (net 23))
 (segment (start 75.635 54.865) (end 75 55.5) (width 0.635) (layer B.Cu) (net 23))
 (segment (start 72.5 58) (end 72.5 66.23) (width 0.635) (layer B.Cu) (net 23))
 (segment (start 75 55.5) (end 72.5 58) (width 0.635) (layer B.Cu) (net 23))
 (segment (start 62.5 66.23) (end 62.5 65.5) (width 0.635) (layer B.Cu) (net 24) (status C00000))
 (segment (start 62.5 65.5) (end 74.405 53.595) (width 0.635) (layer B.Cu) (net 24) (status 400000))
 (segment (start 132.8 53.595) (end 74.405 53.595) (width 0.635) (layer B.Cu) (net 24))
 (segment (start 75 51.055) (end 71.945 51.055) (width 0.381) (layer B.Cu) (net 5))
 (segment (start 59.5 46) (end 60.5 45) (width 0.381) (layer B.Cu) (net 5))
 (segment (start 59.5 52) (end 59.5 46) (width 0.381) (layer B.Cu) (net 5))
 (segment (start 60 52.5) (end 59.5 52) (width 0.381) (layer B.Cu) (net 5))
 (segment (start 70.5 52.5) (end 60 52.5) (width 0.381) (layer B.Cu) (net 5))
 (segment (start 60.5 45) (end 62.5 45) (width 0.381) (layer B.Cu) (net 5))
 (segment (start 71.945 51.055) (end 70.5 52.5) (width 0.381) (layer B.Cu) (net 5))
 (segment (start 132.8 51.055) (end 75 51.055) (width 0.381) (layer B.Cu) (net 5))
 (segment (start 75 51.055) (end 74.945 51.055) (width 0.381) (layer B.Cu) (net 5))
 (segment (start 142.2 49.785) (end 200.215 49.785) (width 0.381) (layer B.Cu) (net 8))
 (segment (start 200.215 49.785) (end 203.5 46.5) (width 0.381) (layer B.Cu) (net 8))
 (segment (start 203.215 46.785) (end 203.5 46.5) (width 0.381) (layer B.Cu) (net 8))
 (segment (start 203.5 46.5) (end 205 45) (width 0.381) (layer B.Cu) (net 8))
 (segment (start 205 45) (end 212.5 45) (width 0.381) (layer B.Cu) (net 8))
 (segment (start 142.2 51.055) (end 201.945 51.055) (width 0.381) (layer B.Cu) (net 4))
 (segment (start 205.5 47.5) (end 212.5 47.5) (width 0.381) (layer B.Cu) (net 4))
 (segment (start 204.945 48.055) (end 205.5 47.5) (width 0.381) (layer B.Cu) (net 4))
 (segment (start 201.945 51.055) (end 204.945 48.055) (width 0.381) (layer B.Cu) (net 4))
 (segment (start 62.5 47.5) (end 68.5 47.5) (width 0.381) (layer B.Cu) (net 4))
 (segment (start 140.055 51.055) (end 142.2 51.055) (width 0.381) (layer B.Cu) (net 4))
 (segment (start 139 50) (end 140.055 51.055) (width 0.381) (layer B.Cu) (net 4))
 (segment (start 139 45.5) (end 139 50) (width 0.381) (layer B.Cu) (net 4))
 (segment (start 137.5 44) (end 139 45.5) (width 0.381) (layer B.Cu) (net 4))
 (segment (start 72 44) (end 137.5 44) (width 0.381) (layer B.Cu) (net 4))
 (segment (start 68.5 47.5) (end 72 44) (width 0.381) (layer B.Cu) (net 4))
 (segment (start 142.2 52.325) (end 204.175 52.325) (width 0.381) (layer B.Cu) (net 3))
 (segment (start 204.175 52.325) (end 206.5 50) (width 0.381) (layer B.Cu) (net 3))
 (segment (start 62.5 50) (end 69.5 50) (width 0.381) (layer B.Cu) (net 3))
 (segment (start 138.825 52.325) (end 142.2 52.325) (width 0.381) (layer B.Cu) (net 3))
 (segment (start 137.5 51) (end 138.825 52.325) (width 0.381) (layer B.Cu) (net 3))
 (segment (start 137.5 46.5) (end 137.5 51) (width 0.381) (layer B.Cu) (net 3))
 (segment (start 136 45) (end 137.5 46.5) (width 0.381) (layer B.Cu) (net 3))
 (segment (start 74.5 45) (end 136 45) (width 0.381) (layer B.Cu) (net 3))
 (segment (start 69.5 50) (end 74.5 45) (width 0.381) (layer B.Cu) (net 3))
 (segment (start 206.5 50) (end 212.5 50) (width 0.381) (layer B.Cu) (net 3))
 (segment (start 137.5 67.5) (end 137.5 54) (width 0.381) (layer B.Cu) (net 2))
 (segment (start 135.825 52.325) (end 137.5 54) (width 0.381) (layer B.Cu) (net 2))
 (segment (start 135.825 52.325) (end 132.8 52.325) (width 0.381) (layer B.Cu) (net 2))
 (segment (start 64 67.5) (end 137.5 67.5) (width 0.381) (layer B.Cu) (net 2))
 (segment (start 137.5 67.5) (end 215 67.5) (width 0.381) (layer B.Cu) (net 2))
 (segment (start 60 67.5) (end 64 67.5) (width 0.381) (layer B.Cu) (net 2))
 (segment (start 215 67.5) (end 215.5 68) (width 0.381) (layer B.Cu) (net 2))
 (segment (start 60.5 72.5) (end 59.5 71.5) (width 0.381) (layer B.Cu) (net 2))
 (segment (start 59.5 71.5) (end 59.5 68) (width 0.381) (layer B.Cu) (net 2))
 (segment (start 59.5 68) (end 60 67.5) (width 0.381) (layer B.Cu) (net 2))
 (segment (start 62.5 72.5) (end 60.5 72.5) (width 0.381) (layer B.Cu) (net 2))
 (segment (start 214.5 72.5) (end 212.5 72.5) (width 0.381) (layer B.Cu) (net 2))
 (segment (start 215.5 71.5) (end 214.5 72.5) (width 0.381) (layer B.Cu) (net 2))
 (segment (start 215.5 68) (end 215.5 71.5) (width 0.381) (layer B.Cu) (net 2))
 (segment (start 132.8 49.785) (end 129.135 49.785) (width 0.635) (layer B.Cu) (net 25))
 (segment (start 129.135 49.785) (end 128.85 49.5) (width 0.635) (layer B.Cu) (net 25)))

